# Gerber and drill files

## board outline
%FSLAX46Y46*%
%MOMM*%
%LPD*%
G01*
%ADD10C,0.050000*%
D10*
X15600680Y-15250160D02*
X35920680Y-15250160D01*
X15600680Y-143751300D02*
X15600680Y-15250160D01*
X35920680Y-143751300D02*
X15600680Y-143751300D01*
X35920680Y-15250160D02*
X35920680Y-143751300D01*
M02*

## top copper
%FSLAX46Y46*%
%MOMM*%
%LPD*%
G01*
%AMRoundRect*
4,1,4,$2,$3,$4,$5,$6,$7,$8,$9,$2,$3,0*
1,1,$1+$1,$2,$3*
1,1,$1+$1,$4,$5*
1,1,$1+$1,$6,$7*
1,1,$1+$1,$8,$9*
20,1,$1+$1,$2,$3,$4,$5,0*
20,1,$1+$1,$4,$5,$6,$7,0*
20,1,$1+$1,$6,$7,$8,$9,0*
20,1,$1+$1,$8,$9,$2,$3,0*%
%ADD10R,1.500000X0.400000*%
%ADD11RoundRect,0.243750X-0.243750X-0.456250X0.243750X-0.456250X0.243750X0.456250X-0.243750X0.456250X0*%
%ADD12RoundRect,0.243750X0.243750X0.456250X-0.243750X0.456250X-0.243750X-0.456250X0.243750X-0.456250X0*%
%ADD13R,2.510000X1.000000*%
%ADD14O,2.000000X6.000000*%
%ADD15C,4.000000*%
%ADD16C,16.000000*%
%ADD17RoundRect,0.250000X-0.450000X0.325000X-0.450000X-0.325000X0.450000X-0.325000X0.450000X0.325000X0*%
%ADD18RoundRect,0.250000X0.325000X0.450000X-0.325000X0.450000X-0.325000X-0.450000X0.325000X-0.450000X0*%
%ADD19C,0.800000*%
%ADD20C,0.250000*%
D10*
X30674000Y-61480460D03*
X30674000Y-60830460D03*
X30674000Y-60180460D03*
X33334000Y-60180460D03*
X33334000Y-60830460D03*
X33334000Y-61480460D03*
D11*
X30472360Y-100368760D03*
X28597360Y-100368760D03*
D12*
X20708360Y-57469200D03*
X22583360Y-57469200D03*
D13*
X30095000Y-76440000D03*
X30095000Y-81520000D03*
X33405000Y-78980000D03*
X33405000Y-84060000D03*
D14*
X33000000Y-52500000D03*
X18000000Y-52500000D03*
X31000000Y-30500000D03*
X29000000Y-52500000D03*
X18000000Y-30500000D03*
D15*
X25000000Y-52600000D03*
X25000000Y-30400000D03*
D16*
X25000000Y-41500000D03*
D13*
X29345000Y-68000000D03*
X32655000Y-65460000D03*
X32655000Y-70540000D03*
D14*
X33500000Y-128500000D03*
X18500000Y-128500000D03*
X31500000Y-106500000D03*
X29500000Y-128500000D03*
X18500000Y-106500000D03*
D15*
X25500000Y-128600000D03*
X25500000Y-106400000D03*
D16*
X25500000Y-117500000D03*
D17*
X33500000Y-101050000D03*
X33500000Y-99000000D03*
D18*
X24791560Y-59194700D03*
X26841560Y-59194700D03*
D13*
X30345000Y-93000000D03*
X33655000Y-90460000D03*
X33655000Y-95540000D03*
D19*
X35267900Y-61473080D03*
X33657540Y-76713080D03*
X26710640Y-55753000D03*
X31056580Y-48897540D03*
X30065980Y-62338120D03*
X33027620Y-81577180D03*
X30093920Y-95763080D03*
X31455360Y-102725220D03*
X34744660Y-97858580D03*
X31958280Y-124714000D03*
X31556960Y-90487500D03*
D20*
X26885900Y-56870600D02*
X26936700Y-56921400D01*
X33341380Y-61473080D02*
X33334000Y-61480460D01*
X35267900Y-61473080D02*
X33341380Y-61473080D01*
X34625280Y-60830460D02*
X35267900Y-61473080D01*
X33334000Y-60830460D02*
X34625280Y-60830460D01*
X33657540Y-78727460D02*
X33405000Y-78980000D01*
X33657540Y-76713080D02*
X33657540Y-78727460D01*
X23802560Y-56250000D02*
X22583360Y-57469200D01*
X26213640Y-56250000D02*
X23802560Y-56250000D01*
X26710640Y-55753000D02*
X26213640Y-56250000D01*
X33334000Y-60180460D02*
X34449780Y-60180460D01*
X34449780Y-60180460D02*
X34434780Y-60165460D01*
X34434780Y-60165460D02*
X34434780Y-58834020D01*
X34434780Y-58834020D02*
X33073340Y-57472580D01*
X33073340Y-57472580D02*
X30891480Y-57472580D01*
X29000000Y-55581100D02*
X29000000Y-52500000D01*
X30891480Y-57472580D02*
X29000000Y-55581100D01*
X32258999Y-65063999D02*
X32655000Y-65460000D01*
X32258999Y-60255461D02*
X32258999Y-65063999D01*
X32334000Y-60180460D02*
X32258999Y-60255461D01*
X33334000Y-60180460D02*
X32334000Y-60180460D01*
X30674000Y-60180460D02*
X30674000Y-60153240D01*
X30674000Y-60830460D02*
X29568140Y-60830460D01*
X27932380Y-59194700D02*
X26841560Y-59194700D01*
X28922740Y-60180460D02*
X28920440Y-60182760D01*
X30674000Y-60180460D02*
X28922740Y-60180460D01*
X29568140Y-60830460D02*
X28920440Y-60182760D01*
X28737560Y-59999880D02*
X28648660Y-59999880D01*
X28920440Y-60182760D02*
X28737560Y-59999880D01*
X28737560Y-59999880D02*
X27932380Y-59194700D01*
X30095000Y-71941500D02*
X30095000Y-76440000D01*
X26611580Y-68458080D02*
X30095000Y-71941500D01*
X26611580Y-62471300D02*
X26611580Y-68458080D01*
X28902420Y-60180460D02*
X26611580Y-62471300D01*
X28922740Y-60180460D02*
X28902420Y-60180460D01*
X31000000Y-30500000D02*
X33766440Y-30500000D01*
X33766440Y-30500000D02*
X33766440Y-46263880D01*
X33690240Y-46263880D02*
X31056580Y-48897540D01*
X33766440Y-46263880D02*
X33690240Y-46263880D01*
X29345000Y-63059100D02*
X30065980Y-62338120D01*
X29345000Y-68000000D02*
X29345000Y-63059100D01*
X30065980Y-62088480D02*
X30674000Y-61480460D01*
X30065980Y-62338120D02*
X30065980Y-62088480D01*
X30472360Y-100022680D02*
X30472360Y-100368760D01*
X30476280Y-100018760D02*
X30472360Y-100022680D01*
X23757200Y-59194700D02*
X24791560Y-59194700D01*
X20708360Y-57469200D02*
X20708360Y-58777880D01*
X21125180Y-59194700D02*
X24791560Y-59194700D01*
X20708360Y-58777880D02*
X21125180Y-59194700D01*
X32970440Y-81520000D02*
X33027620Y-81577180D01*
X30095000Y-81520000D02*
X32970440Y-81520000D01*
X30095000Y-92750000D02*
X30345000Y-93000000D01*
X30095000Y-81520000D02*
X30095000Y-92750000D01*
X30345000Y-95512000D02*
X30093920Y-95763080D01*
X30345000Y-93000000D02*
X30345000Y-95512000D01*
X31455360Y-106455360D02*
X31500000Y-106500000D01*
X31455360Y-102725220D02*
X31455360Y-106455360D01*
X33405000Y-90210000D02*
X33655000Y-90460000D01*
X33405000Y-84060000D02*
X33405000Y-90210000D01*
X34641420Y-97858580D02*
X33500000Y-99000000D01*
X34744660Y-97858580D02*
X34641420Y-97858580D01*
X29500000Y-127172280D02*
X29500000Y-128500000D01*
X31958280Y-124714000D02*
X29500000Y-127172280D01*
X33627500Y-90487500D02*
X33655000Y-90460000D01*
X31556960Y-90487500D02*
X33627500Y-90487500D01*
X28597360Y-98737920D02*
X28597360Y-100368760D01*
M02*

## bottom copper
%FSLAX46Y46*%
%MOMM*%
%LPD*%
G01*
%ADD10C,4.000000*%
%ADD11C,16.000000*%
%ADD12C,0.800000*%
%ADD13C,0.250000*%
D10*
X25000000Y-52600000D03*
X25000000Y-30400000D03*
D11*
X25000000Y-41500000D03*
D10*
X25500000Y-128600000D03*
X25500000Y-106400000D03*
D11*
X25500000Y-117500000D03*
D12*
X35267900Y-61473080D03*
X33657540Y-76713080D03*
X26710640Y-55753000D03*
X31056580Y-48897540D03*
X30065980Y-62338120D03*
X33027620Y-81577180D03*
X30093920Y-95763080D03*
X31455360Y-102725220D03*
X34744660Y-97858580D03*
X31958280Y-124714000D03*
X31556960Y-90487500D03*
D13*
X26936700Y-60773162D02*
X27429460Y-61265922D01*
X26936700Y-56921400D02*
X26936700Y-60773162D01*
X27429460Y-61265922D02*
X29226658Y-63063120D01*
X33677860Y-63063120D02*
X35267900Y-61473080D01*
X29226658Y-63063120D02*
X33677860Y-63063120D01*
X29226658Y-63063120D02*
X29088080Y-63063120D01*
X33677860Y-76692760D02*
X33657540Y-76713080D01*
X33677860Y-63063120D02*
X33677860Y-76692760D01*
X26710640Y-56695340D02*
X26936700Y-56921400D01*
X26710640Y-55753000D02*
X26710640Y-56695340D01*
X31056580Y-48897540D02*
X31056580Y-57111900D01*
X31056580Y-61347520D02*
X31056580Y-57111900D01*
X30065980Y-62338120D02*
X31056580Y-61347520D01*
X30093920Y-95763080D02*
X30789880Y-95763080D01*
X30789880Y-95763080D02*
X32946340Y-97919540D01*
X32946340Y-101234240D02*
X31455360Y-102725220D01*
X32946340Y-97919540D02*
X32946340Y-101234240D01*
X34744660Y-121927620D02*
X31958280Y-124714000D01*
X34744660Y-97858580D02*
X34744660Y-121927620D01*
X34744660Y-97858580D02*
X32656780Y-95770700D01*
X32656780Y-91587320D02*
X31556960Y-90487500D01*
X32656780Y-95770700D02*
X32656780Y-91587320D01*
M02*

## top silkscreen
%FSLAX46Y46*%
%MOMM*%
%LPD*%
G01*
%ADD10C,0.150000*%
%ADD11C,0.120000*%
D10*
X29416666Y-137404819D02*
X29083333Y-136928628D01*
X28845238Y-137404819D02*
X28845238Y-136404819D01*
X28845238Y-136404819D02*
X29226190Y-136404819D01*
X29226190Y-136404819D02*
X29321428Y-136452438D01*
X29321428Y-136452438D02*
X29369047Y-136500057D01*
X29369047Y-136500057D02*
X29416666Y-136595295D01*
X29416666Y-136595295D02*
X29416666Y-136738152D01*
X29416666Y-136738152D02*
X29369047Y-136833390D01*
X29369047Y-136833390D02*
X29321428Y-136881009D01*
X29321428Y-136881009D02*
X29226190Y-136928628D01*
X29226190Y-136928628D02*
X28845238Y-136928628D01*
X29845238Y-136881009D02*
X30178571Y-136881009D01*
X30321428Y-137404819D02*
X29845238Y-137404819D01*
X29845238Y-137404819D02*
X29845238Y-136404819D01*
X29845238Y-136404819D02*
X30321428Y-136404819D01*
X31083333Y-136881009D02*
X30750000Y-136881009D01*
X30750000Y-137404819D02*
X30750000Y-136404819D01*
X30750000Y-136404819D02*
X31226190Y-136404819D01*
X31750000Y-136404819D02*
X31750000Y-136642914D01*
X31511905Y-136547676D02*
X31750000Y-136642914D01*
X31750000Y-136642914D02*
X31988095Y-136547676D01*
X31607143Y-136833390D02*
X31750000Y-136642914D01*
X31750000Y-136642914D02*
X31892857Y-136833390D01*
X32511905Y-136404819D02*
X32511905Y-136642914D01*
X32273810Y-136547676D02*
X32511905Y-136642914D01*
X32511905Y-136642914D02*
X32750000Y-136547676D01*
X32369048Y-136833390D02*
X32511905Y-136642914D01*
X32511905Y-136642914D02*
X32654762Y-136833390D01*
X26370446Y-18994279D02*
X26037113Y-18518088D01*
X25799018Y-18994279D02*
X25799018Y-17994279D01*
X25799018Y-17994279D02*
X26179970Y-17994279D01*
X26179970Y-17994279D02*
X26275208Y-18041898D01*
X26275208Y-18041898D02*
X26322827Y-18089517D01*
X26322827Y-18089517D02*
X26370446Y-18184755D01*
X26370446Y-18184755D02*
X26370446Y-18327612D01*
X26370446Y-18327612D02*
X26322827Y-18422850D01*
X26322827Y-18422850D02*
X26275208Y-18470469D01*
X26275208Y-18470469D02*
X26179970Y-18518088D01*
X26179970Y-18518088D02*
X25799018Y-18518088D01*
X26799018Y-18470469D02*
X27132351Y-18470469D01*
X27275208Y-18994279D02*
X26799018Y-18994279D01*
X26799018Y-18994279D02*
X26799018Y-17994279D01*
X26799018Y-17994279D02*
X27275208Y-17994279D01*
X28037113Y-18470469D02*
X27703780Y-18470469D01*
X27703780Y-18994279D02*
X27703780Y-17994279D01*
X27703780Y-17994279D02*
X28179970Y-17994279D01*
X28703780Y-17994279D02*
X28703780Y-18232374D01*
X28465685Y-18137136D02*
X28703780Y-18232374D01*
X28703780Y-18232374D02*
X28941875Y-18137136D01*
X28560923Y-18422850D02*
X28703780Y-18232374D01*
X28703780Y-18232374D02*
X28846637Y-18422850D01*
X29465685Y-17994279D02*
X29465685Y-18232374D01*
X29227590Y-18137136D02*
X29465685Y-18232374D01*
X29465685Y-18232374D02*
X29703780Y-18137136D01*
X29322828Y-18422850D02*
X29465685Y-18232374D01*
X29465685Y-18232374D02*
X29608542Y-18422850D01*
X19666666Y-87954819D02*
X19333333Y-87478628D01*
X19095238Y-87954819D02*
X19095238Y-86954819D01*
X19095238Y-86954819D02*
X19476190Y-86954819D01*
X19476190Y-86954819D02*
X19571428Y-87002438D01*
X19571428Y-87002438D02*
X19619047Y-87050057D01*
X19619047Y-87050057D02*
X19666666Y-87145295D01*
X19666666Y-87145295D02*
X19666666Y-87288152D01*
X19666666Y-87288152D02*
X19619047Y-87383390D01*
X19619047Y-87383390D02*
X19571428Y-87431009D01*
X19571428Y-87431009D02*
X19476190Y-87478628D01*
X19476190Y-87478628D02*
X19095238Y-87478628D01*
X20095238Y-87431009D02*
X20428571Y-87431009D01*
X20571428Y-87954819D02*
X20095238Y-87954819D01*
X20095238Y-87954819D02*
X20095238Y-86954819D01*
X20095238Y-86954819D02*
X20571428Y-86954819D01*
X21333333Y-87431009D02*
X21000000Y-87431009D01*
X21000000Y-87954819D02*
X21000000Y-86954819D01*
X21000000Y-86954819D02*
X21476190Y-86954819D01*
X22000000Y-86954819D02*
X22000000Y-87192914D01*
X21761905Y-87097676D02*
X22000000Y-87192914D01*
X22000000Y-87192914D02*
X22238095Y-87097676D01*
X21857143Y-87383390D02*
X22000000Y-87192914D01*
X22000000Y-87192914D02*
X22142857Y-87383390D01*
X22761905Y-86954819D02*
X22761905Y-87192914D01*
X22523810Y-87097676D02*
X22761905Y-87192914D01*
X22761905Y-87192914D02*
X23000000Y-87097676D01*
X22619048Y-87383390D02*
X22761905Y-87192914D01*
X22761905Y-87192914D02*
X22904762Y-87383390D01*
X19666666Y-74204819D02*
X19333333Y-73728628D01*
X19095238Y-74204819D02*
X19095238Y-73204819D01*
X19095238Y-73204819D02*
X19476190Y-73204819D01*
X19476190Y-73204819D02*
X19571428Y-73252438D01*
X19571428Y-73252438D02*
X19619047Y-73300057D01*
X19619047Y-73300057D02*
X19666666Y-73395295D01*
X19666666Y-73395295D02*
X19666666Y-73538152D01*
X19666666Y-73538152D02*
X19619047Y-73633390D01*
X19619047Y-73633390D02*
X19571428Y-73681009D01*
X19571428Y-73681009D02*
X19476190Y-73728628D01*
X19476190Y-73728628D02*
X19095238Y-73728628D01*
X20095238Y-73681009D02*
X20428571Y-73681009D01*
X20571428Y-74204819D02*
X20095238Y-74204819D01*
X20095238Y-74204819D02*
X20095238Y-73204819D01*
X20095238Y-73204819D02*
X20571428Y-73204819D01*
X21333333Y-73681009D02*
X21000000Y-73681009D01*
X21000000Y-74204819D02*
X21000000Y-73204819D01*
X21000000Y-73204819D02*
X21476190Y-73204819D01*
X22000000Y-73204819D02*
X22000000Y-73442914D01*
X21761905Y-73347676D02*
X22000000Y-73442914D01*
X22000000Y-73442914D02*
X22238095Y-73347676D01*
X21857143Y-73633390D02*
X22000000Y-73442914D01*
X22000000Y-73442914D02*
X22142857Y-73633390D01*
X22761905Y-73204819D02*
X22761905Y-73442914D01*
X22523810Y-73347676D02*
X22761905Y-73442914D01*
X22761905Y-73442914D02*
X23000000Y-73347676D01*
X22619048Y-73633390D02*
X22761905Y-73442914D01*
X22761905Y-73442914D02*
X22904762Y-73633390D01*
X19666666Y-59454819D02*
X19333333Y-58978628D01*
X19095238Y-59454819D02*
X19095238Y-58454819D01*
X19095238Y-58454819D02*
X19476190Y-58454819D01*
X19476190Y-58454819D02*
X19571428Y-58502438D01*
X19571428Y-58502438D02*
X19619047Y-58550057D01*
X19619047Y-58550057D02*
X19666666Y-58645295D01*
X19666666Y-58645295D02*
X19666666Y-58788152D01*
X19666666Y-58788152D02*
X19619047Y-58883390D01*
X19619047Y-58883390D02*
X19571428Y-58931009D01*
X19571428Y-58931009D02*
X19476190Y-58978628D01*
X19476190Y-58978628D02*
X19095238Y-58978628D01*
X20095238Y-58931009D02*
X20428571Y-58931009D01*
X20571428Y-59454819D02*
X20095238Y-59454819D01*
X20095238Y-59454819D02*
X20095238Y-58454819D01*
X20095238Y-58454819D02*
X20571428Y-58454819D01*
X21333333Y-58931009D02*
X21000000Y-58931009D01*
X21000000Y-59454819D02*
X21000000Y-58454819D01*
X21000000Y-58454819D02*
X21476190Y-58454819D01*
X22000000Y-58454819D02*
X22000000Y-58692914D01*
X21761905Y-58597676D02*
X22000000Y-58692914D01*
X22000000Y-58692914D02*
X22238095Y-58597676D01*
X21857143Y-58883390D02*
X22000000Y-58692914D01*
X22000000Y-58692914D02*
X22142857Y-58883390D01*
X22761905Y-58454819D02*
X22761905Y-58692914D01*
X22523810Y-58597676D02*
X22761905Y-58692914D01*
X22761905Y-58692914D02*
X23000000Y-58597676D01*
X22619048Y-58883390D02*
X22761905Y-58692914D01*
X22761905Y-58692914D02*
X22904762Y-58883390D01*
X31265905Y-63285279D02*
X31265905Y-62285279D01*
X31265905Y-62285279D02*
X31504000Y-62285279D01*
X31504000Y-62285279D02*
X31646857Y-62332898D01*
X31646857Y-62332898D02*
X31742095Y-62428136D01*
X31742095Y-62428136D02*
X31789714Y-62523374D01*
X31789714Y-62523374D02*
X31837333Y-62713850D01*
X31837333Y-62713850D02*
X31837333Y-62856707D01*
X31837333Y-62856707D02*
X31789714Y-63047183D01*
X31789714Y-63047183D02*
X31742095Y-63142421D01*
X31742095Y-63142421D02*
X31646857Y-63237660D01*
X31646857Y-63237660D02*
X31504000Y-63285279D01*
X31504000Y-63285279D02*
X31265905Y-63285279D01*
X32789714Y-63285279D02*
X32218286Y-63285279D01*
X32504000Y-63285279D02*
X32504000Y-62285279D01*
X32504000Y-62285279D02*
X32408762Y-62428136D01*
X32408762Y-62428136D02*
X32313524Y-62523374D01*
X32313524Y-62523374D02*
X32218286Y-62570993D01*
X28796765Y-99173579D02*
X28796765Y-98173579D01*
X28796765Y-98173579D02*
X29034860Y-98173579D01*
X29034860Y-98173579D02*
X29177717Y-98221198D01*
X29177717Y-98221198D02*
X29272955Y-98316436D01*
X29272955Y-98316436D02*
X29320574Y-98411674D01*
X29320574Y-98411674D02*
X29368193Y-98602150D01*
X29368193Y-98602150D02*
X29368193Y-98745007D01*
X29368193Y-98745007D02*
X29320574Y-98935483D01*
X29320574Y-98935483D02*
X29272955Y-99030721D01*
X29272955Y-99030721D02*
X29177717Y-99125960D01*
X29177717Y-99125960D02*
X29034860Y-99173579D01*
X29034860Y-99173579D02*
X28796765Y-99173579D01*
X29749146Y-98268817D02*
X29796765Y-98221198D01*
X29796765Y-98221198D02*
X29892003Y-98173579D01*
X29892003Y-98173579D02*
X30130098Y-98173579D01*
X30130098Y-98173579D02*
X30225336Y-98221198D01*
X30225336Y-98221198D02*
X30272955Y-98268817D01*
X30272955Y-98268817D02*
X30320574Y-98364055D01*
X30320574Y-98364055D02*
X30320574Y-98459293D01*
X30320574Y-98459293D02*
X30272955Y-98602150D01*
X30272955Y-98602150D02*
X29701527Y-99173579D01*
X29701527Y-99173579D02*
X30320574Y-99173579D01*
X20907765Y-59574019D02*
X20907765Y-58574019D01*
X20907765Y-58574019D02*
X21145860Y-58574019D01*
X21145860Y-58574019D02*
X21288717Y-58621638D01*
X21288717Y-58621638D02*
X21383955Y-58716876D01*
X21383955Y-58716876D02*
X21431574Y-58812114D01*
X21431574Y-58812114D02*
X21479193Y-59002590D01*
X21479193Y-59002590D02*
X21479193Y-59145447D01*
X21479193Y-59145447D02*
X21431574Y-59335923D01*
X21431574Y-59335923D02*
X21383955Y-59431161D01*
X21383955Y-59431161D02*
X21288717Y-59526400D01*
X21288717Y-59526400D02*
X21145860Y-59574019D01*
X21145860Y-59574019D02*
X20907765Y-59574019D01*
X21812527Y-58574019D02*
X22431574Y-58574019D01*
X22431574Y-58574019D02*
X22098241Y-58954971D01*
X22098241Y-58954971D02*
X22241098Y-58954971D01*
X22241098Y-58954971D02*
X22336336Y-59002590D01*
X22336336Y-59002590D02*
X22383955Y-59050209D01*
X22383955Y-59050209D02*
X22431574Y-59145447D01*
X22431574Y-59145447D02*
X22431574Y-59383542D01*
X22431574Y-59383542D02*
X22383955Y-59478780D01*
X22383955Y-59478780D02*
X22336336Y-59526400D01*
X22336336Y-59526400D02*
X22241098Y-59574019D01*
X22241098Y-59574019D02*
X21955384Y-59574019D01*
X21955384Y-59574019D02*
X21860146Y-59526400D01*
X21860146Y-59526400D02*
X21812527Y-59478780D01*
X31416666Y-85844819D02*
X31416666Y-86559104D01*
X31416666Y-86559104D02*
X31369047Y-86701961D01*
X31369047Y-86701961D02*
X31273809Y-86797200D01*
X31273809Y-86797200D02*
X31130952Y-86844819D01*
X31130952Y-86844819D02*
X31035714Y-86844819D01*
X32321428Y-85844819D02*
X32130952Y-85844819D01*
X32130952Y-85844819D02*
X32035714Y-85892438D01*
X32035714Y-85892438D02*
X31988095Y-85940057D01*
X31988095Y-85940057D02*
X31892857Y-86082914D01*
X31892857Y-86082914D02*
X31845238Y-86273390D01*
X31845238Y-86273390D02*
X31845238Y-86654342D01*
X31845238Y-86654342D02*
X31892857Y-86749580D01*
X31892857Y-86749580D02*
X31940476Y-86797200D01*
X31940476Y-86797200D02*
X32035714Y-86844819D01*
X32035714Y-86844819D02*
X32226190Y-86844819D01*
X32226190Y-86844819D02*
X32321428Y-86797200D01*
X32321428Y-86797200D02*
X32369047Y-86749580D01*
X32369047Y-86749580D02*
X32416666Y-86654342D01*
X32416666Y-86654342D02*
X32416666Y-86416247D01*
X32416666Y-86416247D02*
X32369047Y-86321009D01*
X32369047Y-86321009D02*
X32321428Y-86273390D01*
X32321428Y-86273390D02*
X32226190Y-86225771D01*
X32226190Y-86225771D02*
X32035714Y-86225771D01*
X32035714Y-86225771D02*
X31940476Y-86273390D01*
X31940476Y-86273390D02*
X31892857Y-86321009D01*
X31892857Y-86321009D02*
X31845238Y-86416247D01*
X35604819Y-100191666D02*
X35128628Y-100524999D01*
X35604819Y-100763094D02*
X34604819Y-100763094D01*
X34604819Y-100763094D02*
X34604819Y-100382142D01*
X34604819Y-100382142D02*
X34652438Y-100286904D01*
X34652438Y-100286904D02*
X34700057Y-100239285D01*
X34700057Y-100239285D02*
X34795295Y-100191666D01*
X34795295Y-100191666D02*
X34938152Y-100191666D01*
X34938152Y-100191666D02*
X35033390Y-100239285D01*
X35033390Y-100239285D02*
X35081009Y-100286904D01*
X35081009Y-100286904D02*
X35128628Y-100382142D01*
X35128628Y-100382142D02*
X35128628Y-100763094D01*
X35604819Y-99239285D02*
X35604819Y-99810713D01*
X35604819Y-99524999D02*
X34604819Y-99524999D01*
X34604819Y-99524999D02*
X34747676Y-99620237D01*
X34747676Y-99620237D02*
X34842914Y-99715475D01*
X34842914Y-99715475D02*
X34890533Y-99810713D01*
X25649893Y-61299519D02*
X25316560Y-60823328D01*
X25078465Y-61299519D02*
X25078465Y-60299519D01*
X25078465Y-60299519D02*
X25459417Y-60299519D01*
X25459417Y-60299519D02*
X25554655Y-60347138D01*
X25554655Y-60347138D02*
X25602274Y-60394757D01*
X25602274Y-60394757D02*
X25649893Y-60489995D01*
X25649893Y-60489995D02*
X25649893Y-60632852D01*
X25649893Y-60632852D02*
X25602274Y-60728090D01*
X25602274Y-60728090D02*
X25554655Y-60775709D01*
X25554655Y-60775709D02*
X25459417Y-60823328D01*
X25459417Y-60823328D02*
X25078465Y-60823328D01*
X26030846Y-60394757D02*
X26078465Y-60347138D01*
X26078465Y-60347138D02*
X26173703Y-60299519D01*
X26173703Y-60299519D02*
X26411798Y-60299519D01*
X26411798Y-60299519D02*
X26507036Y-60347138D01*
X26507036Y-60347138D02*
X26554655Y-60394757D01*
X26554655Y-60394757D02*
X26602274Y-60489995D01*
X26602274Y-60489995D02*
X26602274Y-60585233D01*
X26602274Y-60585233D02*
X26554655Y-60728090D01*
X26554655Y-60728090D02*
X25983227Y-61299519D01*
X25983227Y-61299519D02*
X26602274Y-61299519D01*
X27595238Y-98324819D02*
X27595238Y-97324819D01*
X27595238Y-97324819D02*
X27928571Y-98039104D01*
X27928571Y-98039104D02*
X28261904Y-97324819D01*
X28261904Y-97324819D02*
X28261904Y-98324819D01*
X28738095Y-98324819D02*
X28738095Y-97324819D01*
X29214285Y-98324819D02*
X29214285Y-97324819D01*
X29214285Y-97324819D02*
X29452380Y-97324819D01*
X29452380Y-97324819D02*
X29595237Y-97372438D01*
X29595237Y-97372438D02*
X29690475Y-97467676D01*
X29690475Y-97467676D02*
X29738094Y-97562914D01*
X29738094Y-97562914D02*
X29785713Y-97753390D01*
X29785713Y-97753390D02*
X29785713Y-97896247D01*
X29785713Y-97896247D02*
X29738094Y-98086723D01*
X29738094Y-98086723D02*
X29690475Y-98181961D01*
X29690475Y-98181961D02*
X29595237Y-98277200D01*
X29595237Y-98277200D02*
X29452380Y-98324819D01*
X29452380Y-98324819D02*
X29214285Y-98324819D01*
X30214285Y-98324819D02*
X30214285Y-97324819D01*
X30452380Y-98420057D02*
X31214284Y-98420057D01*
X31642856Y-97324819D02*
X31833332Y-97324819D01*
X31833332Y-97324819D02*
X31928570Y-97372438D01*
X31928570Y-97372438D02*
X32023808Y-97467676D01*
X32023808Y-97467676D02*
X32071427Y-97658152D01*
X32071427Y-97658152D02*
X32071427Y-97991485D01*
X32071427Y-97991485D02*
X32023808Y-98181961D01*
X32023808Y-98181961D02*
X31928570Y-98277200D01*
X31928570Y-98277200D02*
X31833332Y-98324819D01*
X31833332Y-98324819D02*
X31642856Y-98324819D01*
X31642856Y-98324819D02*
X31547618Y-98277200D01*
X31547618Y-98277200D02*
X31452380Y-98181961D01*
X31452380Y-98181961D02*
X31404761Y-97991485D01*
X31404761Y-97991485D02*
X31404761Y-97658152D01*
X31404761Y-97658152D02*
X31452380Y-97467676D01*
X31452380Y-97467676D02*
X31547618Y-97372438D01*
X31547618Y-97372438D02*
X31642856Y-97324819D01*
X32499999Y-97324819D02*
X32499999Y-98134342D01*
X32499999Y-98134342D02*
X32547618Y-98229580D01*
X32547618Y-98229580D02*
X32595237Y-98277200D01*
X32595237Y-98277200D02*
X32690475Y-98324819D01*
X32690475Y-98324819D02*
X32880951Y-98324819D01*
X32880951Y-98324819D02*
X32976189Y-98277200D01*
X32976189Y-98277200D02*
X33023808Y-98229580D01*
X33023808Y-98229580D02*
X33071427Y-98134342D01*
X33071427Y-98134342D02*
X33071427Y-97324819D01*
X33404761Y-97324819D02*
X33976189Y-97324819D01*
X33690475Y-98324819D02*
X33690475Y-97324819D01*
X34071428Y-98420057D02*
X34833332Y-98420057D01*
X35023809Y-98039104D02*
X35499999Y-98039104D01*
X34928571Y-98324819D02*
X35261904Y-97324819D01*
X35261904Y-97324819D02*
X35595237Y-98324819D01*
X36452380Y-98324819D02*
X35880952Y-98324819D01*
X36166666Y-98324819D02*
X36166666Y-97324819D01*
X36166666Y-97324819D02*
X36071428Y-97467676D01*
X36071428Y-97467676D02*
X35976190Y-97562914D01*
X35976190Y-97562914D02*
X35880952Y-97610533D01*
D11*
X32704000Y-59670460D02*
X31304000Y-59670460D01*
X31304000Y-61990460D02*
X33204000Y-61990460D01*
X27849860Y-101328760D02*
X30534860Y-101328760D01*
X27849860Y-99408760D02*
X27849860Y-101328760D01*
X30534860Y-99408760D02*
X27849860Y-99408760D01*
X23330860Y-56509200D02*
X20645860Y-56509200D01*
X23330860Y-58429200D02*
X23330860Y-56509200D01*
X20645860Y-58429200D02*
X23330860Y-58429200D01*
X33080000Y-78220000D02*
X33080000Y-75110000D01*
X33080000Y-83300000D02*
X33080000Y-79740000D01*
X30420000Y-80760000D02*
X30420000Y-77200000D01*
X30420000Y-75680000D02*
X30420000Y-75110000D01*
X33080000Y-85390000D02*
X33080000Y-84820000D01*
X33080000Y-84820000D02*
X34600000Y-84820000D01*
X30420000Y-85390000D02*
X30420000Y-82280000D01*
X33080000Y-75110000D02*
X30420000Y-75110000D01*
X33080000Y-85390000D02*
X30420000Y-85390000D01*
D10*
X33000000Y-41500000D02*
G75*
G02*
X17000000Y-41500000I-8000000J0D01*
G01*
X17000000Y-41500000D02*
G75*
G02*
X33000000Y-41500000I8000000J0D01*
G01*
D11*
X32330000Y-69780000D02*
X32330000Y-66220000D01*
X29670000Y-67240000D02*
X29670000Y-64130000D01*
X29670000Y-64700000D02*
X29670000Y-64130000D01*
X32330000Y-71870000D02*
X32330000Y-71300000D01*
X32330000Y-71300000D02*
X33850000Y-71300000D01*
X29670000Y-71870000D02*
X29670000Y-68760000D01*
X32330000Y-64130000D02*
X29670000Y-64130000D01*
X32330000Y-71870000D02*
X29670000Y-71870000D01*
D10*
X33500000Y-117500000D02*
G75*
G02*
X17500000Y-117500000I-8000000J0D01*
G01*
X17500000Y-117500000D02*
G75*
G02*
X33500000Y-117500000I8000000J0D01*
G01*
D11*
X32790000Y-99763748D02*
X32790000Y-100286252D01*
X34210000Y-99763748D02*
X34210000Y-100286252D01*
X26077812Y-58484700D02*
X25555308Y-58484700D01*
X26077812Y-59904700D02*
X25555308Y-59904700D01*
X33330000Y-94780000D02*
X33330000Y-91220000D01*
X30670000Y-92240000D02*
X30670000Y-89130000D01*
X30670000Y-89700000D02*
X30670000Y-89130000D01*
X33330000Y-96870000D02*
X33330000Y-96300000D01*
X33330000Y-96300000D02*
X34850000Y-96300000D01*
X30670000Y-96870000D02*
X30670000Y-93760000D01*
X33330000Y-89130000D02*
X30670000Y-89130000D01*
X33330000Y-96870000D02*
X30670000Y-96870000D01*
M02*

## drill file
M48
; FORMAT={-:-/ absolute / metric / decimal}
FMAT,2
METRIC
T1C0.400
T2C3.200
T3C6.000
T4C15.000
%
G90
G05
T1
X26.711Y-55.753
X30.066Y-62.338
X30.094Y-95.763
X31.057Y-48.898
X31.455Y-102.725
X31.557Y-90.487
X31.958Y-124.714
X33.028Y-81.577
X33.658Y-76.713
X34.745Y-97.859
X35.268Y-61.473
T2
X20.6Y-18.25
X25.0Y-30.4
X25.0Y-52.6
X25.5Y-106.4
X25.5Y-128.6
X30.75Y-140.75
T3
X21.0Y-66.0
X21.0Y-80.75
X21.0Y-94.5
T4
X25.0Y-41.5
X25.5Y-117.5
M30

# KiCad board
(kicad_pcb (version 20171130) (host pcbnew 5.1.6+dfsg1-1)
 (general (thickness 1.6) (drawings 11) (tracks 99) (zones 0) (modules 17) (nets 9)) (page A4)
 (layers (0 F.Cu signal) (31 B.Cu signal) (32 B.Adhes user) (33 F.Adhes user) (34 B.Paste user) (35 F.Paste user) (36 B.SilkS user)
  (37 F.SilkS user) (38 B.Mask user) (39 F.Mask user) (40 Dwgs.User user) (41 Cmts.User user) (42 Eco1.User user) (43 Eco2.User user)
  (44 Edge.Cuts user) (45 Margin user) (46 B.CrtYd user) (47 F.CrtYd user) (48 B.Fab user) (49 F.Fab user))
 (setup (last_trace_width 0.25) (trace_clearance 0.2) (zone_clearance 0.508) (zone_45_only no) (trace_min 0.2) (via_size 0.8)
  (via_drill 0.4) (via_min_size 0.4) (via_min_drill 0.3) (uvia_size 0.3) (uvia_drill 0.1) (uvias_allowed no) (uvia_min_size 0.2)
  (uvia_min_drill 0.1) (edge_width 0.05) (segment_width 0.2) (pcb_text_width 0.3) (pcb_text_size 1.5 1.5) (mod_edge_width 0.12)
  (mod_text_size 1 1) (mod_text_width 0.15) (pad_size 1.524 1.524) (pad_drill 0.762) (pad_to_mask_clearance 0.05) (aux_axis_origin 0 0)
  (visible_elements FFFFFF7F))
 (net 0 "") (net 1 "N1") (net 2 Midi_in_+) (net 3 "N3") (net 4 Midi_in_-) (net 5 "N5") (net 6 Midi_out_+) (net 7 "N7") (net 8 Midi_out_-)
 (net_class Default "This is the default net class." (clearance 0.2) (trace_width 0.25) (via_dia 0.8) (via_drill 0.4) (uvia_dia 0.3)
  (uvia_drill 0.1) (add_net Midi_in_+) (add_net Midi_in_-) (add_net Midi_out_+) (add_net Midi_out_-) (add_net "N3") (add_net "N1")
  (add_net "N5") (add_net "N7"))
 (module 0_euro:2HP (layer F.Cu) (at 15.6 15)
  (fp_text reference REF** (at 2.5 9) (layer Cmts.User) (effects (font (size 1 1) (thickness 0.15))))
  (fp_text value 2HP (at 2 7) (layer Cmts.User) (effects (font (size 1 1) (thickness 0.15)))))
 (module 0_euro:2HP (layer F.Cu) (at 25.76 15)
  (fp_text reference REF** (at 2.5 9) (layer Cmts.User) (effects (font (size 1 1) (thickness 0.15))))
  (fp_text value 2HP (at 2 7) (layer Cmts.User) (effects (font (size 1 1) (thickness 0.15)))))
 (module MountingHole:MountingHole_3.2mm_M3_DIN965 (layer F.Cu) (at 30.75 140.75)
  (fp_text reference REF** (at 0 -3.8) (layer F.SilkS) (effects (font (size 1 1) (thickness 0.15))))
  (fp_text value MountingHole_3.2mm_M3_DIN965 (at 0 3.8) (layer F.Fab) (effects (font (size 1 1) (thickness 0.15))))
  (pad 1 np_thru_hole circle (at 0 0) (size 3.2 3.2) (drill 3.2) (layers *.Cu *.Mask)))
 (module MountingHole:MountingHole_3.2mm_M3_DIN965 (layer F.Cu) (at 20.6 18.25)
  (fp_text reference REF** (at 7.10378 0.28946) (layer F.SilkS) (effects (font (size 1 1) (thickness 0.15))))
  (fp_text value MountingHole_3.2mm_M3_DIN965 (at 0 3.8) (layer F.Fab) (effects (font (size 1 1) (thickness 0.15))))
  (pad 1 np_thru_hole circle (at 0 0) (size 3.2 3.2) (drill 3.2) (layers *.Cu *.Mask)))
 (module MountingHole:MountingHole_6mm (layer F.Cu) (at 21 94.5)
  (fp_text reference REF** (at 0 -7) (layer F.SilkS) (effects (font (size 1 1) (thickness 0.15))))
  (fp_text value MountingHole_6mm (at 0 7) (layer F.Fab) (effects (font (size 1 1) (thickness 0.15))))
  (pad 1 np_thru_hole circle (at 0 0) (size 6 6) (drill 6) (layers *.Cu *.Mask)))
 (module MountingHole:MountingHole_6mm (layer F.Cu) (at 21 80.75)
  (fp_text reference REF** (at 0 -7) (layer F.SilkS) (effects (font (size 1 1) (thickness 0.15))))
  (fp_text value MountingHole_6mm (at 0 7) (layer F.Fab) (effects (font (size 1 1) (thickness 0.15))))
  (pad 1 np_thru_hole circle (at 0 0) (size 6 6) (drill 6) (layers *.Cu *.Mask)))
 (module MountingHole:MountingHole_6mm (layer F.Cu) (at 21 66)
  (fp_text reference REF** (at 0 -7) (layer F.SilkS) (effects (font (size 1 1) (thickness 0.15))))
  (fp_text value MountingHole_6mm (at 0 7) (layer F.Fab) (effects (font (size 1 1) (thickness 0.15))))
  (pad 1 np_thru_hole circle (at 0 0) (size 6 6) (drill 6) (layers *.Cu *.Mask)))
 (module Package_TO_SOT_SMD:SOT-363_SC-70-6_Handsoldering (layer F.Cu) (at 32.004 60.83046 180)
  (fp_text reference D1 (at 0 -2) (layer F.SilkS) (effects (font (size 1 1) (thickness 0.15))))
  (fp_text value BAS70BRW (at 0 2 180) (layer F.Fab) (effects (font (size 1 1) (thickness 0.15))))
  (fp_line (start -0.7 1.16) (end 0.7 1.16) (layer F.SilkS) (width 0.12))
  (fp_line (start 0.7 -1.16) (end -1.2 -1.16) (layer F.SilkS) (width 0.12))
  (pad 6 smd rect (at 1.33 -0.65 180) (size 1.5 0.4) (layers F.Cu F.Paste F.Mask) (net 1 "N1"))
  (pad 5 smd rect (at 1.33 0 180) (size 1.5 0.4) (layers F.Cu F.Paste F.Mask) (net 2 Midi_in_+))
  (pad 4 smd rect (at 1.33 0.65 180) (size 1.5 0.4) (layers F.Cu F.Paste F.Mask) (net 2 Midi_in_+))
  (pad 3 smd rect (at -1.33 0.65 180) (size 1.5 0.4) (layers F.Cu F.Paste F.Mask) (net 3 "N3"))
  (pad 2 smd rect (at -1.33 0 180) (size 1.5 0.4) (layers F.Cu F.Paste F.Mask) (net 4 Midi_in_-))
  (pad 1 smd rect (at -1.33 -0.65 180) (size 1.5 0.4) (layers F.Cu F.Paste F.Mask) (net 4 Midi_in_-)))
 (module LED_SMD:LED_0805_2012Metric (layer F.Cu) (at 29.53486 100.36876)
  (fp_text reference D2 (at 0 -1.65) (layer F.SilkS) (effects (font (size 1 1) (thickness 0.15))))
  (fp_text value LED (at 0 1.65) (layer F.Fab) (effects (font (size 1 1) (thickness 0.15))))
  (fp_line (start -1.685 0.96) (end 1 0.96) (layer F.SilkS) (width 0.12))
  (fp_line (start -1.685 -0.96) (end -1.685 0.96) (layer F.SilkS) (width 0.12))
  (fp_line (start 1 -0.96) (end -1.685 -0.96) (layer F.SilkS) (width 0.12))
  (pad 2 smd roundrect (at 0.9375 0) (size 0.975 1.4) (layers F.Cu F.Paste F.Mask) (roundrect_rratio 0.25) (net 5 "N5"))
  (pad 1 smd roundrect (at -0.9375 0) (size 0.975 1.4) (layers F.Cu F.Paste F.Mask) (roundrect_rratio 0.25) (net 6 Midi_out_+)))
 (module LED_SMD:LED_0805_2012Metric (layer F.Cu) (at 21.64586 57.4692 180)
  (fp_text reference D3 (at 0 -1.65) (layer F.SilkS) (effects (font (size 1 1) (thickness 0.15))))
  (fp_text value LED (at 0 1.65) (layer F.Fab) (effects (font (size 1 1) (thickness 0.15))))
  (fp_line (start -1.685 0.96) (end 1 0.96) (layer F.SilkS) (width 0.12))
  (fp_line (start -1.685 -0.96) (end -1.685 0.96) (layer F.SilkS) (width 0.12))
  (fp_line (start 1 -0.96) (end -1.685 -0.96) (layer F.SilkS) (width 0.12))
  (pad 2 smd roundrect (at 0.9375 0 180) (size 0.975 1.4) (layers F.Cu F.Paste F.Mask) (roundrect_rratio 0.25) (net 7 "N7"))
  (pad 1 smd roundrect (at -0.9375 0 180) (size 0.975 1.4) (layers F.Cu F.Paste F.Mask) (roundrect_rratio 0.25) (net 4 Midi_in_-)))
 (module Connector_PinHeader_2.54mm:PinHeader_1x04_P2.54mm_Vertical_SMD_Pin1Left (layer F.Cu) (at 31.75 80.25 180)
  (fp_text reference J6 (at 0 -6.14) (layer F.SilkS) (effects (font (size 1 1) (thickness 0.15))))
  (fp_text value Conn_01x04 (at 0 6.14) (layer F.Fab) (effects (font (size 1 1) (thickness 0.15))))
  (fp_line (start -1.33 2.03) (end -1.33 5.14) (layer F.SilkS) (width 0.12))
  (fp_line (start -1.33 -3.05) (end -1.33 0.51) (layer F.SilkS) (width 0.12))
  (fp_line (start 1.33 -0.51) (end 1.33 3.05) (layer F.SilkS) (width 0.12))
  (fp_line (start 1.33 4.57) (end 1.33 5.14) (layer F.SilkS) (width 0.12))
  (fp_line (start -1.33 -5.14) (end -1.33 -4.57) (layer F.SilkS) (width 0.12))
  (fp_line (start -1.33 -4.57) (end -2.85 -4.57) (layer F.SilkS) (width 0.12))
  (fp_line (start 1.33 -5.14) (end 1.33 -2.03) (layer F.SilkS) (width 0.12))
  (fp_line (start -1.33 5.14) (end 1.33 5.14) (layer F.SilkS) (width 0.12))
  (fp_line (start -1.33 -5.14) (end 1.33 -5.14) (layer F.SilkS) (width 0.12))
  (pad 4 smd rect (at 1.655 3.81 180) (size 2.51 1) (layers F.Cu F.Paste F.Mask) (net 2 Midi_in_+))
  (pad 2 smd rect (at 1.655 -1.27 180) (size 2.51 1) (layers F.Cu F.Paste F.Mask) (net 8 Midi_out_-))
  (pad 3 smd rect (at -1.655 1.27 180) (size 2.51 1) (layers F.Cu F.Paste F.Mask) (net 4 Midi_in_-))
  (pad 1 smd rect (at -1.655 -3.81 180) (size 2.51 1) (layers F.Cu F.Paste F.Mask) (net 6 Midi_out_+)))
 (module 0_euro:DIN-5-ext (layer F.Cu) (at 25 41.5)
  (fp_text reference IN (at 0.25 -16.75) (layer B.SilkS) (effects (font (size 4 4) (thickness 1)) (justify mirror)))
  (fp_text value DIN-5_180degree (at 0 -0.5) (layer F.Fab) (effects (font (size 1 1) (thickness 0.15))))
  (fp_circle (center 0 0) (end 0 -8) (layer F.SilkS) (width 0.15))
  (pad 2 smd oval (at 8 11) (size 2 6) (layers F.Cu F.Paste F.Mask))
  (pad 1 smd oval (at -7 11) (size 2 6) (layers F.Cu F.Paste F.Mask))
  (pad 5 smd oval (at 6 -11) (size 2 6) (layers F.Cu F.Paste F.Mask) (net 1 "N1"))
  (pad 4 smd oval (at 4 11) (size 2 6) (layers F.Cu F.Paste F.Mask) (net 3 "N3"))
  (pad 3 smd oval (at -7 -11) (size 2 6) (layers F.Cu F.Paste F.Mask))
  (pad "" np_thru_hole circle (at 0 11.1) (size 4 4) (drill 3.2) (layers *.Cu *.Mask))
  (pad "" np_thru_hole circle (at 0 -11.1) (size 4 4) (drill 3.2) (layers *.Cu *.Mask))
  (pad "" np_thru_hole circle (at 0 0) (size 16 16) (drill 15) (layers *.Cu *.Mask)))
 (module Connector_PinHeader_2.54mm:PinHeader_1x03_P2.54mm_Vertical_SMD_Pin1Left (layer F.Cu) (at 31 68 180)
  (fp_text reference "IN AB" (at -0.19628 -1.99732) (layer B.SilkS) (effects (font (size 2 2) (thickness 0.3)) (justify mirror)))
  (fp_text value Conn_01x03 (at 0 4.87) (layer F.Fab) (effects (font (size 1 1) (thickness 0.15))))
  (fp_line (start -1.33 -1.78) (end -1.33 1.78) (layer F.SilkS) (width 0.12))
  (fp_line (start 1.33 0.76) (end 1.33 3.87) (layer F.SilkS) (width 0.12))
  (fp_line (start 1.33 3.3) (end 1.33 3.87) (layer F.SilkS) (width 0.12))
  (fp_line (start -1.33 -3.87) (end -1.33 -3.3) (layer F.SilkS) (width 0.12))
  (fp_line (start -1.33 -3.3) (end -2.85 -3.3) (layer F.SilkS) (width 0.12))
  (fp_line (start 1.33 -3.87) (end 1.33 -0.76) (layer F.SilkS) (width 0.12))
  (fp_line (start -1.33 3.87) (end 1.33 3.87) (layer F.SilkS) (width 0.12))
  (fp_line (start -1.33 -3.87) (end 1.33 -3.87) (layer F.SilkS) (width 0.12))
  (pad 2 smd rect (at 1.655 0 180) (size 2.51 1) (layers F.Cu F.Paste F.Mask) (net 1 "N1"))
  (pad 3 smd rect (at -1.655 2.54 180) (size 2.51 1) (layers F.Cu F.Paste F.Mask) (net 3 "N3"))
  (pad 1 smd rect (at -1.655 -2.54 180) (size 2.51 1) (layers F.Cu F.Paste F.Mask)))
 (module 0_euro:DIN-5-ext (layer F.Cu) (at 25.5 117.5)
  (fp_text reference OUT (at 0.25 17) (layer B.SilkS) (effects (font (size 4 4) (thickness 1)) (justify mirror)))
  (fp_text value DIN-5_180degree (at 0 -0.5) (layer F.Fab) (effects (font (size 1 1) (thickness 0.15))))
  (fp_circle (center 0 0) (end 0 -8) (layer F.SilkS) (width 0.15))
  (pad 2 smd oval (at 8 11) (size 2 6) (layers F.Cu F.Paste F.Mask))
  (pad 1 smd oval (at -7 11) (size 2 6) (layers F.Cu F.Paste F.Mask))
  (pad 5 smd oval (at 6 -11) (size 2 6) (layers F.Cu F.Paste F.Mask) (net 8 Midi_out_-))
  (pad 4 smd oval (at 4 11) (size 2 6) (layers F.Cu F.Paste F.Mask) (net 6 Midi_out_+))
  (pad 3 smd oval (at -7 -11) (size 2 6) (layers F.Cu F.Paste F.Mask))
  (pad "" np_thru_hole circle (at 0 11.1) (size 4 4) (drill 3.2) (layers *.Cu *.Mask))
  (pad "" np_thru_hole circle (at 0 -11.1) (size 4 4) (drill 3.2) (layers *.Cu *.Mask))
  (pad "" np_thru_hole circle (at 0 0) (size 16 16) (drill 15) (layers *.Cu *.Mask)))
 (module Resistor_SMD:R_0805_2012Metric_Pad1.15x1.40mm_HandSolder (layer F.Cu) (at 33.5 100.025 270)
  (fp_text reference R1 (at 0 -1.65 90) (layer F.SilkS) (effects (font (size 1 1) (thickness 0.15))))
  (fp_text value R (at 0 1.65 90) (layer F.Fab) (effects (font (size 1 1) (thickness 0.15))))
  (fp_line (start -0.261252 0.71) (end 0.261252 0.71) (layer F.SilkS) (width 0.12))
  (fp_line (start -0.261252 -0.71) (end 0.261252 -0.71) (layer F.SilkS) (width 0.12))
  (pad 2 smd roundrect (at 1.025 0 270) (size 1.15 1.4) (layers F.Cu F.Paste F.Mask) (roundrect_rratio 0.217391) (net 5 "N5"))
  (pad 1 smd roundrect (at -1.025 0 270) (size 1.15 1.4) (layers F.Cu F.Paste F.Mask) (roundrect_rratio 0.217391) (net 6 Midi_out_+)))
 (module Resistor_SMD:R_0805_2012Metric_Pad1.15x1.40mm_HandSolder (layer F.Cu) (at 25.81656 59.1947 180)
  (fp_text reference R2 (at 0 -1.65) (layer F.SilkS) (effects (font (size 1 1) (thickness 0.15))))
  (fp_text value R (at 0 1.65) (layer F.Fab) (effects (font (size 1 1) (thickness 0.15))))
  (fp_line (start -0.261252 0.71) (end 0.261252 0.71) (layer F.SilkS) (width 0.12))
  (fp_line (start -0.261252 -0.71) (end 0.261252 -0.71) (layer F.SilkS) (width 0.12))
  (pad 2 smd roundrect (at 1.025 0 180) (size 1.15 1.4) (layers F.Cu F.Paste F.Mask) (roundrect_rratio 0.217391) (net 7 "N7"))
  (pad 1 smd roundrect (at -1.025 0 180) (size 1.15 1.4) (layers F.Cu F.Paste F.Mask) (roundrect_rratio 0.217391) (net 2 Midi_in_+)))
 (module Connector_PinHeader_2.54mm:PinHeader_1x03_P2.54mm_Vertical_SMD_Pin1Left (layer F.Cu) (at 32 93 180)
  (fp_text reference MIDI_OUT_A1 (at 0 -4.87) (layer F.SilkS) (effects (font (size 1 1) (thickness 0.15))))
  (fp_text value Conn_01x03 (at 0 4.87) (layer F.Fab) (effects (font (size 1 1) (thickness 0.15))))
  (fp_line (start -1.33 -1.78) (end -1.33 1.78) (layer F.SilkS) (width 0.12))
  (fp_line (start 1.33 0.76) (end 1.33 3.87) (layer F.SilkS) (width 0.12))
  (fp_line (start 1.33 3.3) (end 1.33 3.87) (layer F.SilkS) (width 0.12))
  (fp_line (start -1.33 -3.87) (end -1.33 -3.3) (layer F.SilkS) (width 0.12))
  (fp_line (start -1.33 -3.3) (end -2.85 -3.3) (layer F.SilkS) (width 0.12))
  (fp_line (start 1.33 -3.87) (end 1.33 -0.76) (layer F.SilkS) (width 0.12))
  (fp_line (start -1.33 3.87) (end 1.33 3.87) (layer F.SilkS) (width 0.12))
  (fp_line (start -1.33 -3.87) (end 1.33 -3.87) (layer F.SilkS) (width 0.12))
  (pad 2 smd rect (at 1.655 0 180) (size 2.51 1) (layers F.Cu F.Paste F.Mask) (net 8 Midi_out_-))
  (pad 3 smd rect (at -1.655 2.54 180) (size 2.51 1) (layers F.Cu F.Paste F.Mask) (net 6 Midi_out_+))
  (pad 1 smd rect (at -1.655 -2.54 180) (size 2.51 1) (layers F.Cu F.Paste F.Mask)))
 (gr_line (start 15.60068 15.25016) (end 35.92068 15.25016) (layer Edge.Cuts) (width 0.05))
 (gr_line (start 15.60068 143.7513) (end 15.60068 15.25016) (layer Edge.Cuts) (width 0.05))
 (gr_line (start 35.92068 143.7513) (end 15.60068 143.7513) (layer Edge.Cuts) (width 0.05))
 (gr_line (start 35.92068 15.25016) (end 35.92068 143.7513) (layer Edge.Cuts) (width 0.05))
 (segment (start 26.8859 56.8706) (end 26.9367 56.9214) (width 0.25) (layer F.Cu) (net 4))
 (segment (start 26.9367 60.773162) (end 27.42946 61.265922) (width 0.25) (layer B.Cu) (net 4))
 (segment (start 26.9367 56.9214) (end 26.9367 60.773162) (width 0.25) (layer B.Cu) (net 4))
 (segment (start 27.42946 61.265922) (end 29.226658 63.06312) (width 0.25) (layer B.Cu) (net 4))
 (via (at 35.2679 61.47308) (size 0.8) (drill 0.4) (layers F.Cu B.Cu) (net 4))
 (segment (start 33.67786 63.06312) (end 35.2679 61.47308) (width 0.25) (layer B.Cu) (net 4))
 (segment (start 29.226658 63.06312) (end 33.67786 63.06312) (width 0.25) (layer B.Cu) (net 4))
 (segment (start 33.34138 61.47308) (end 33.334 61.48046) (width 0.25) (layer F.Cu) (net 4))
 (segment (start 35.2679 61.47308) (end 33.34138 61.47308) (width 0.25) (layer F.Cu) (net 4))
 (segment (start 34.62528 60.83046) (end 35.2679 61.47308) (width 0.25) (layer F.Cu) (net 4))
 (segment (start 33.334 60.83046) (end 34.62528 60.83046) (width 0.25) (layer F.Cu) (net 4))
 (segment (start 29.226658 63.06312) (end 29.08808 63.06312) (width 0.25) (layer B.Cu) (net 4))
 (via (at 33.65754 76.71308) (size 0.8) (drill 0.4) (layers F.Cu B.Cu) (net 4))
 (segment (start 33.67786 76.69276) (end 33.65754 76.71308) (width 0.25) (layer B.Cu) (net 4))
 (segment (start 33.67786 63.06312) (end 33.67786 76.69276) (width 0.25) (layer B.Cu) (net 4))
 (segment (start 33.65754 78.72746) (end 33.405 78.98) (width 0.25) (layer F.Cu) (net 4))
 (segment (start 33.65754 76.71308) (end 33.65754 78.72746) (width 0.25) (layer F.Cu) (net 4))
 (via (at 26.71064 55.753) (size 0.8) (drill 0.4) (layers F.Cu B.Cu) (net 4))
 (segment (start 26.71064 56.69534) (end 26.9367 56.9214) (width 0.25) (layer B.Cu) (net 4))
 (segment (start 26.71064 55.753) (end 26.71064 56.69534) (width 0.25) (layer B.Cu) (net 4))
 (segment (start 23.80256 56.25) (end 22.58336 57.4692) (width 0.25) (layer F.Cu) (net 4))
 (segment (start 26.21364 56.25) (end 23.80256 56.25) (width 0.25) (layer F.Cu) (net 4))
 (segment (start 26.71064 55.753) (end 26.21364 56.25) (width 0.25) (layer F.Cu) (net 4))
 (segment (start 33.334 60.18046) (end 34.44978 60.18046) (width 0.25) (layer F.Cu) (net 3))
 (segment (start 34.44978 60.18046) (end 34.43478 60.16546) (width 0.25) (layer F.Cu) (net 3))
 (segment (start 34.43478 60.16546) (end 34.43478 58.83402) (width 0.25) (layer F.Cu) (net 3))
 (segment (start 34.43478 58.83402) (end 33.07334 57.47258) (width 0.25) (layer F.Cu) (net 3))
 (segment (start 33.07334 57.47258) (end 30.89148 57.47258) (width 0.25) (layer F.Cu) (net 3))
 (segment (start 29 55.5811) (end 29 52.5) (width 0.25) (layer F.Cu) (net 3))
 (segment (start 30.89148 57.47258) (end 29 55.5811) (width 0.25) (layer F.Cu) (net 3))
 (segment (start 32.258999 65.063999) (end 32.655 65.46) (width 0.25) (layer F.Cu) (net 3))
 (segment (start 32.258999 60.255461) (end 32.258999 65.063999) (width 0.25) (layer F.Cu) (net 3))
 (segment (start 32.334 60.18046) (end 32.258999 60.255461) (width 0.25) (layer F.Cu) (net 3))
 (segment (start 33.334 60.18046) (end 32.334 60.18046) (width 0.25) (layer F.Cu) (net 3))
 (segment (start 30.674 60.18046) (end 30.674 60.15324) (width 0.25) (layer F.Cu) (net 2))
 (segment (start 30.674 60.83046) (end 29.56814 60.83046) (width 0.25) (layer F.Cu) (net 2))
 (segment (start 27.93238 59.1947) (end 26.84156 59.1947) (width 0.25) (layer F.Cu) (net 2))
 (segment (start 28.92274 60.18046) (end 28.92044 60.18276) (width 0.25) (layer F.Cu) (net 2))
 (segment (start 30.674 60.18046) (end 28.92274 60.18046) (width 0.25) (layer F.Cu) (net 2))
 (segment (start 29.56814 60.83046) (end 28.92044 60.18276) (width 0.25) (layer F.Cu) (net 2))
 (segment (start 28.73756 59.99988) (end 28.64866 59.99988) (width 0.25) (layer F.Cu) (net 2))
 (segment (start 28.92044 60.18276) (end 28.73756 59.99988) (width 0.25) (layer F.Cu) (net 2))
 (segment (start 28.73756 59.99988) (end 27.93238 59.1947) (width 0.25) (layer F.Cu) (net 2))
 (segment (start 30.095 71.9415) (end 30.095 76.44) (width 0.25) (layer F.Cu) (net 2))
 (segment (start 26.61158 68.45808) (end 30.095 71.9415) (width 0.25) (layer F.Cu) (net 2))
 (segment (start 26.61158 62.4713) (end 26.61158 68.45808) (width 0.25) (layer F.Cu) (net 2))
 (segment (start 28.90242 60.18046) (end 26.61158 62.4713) (width 0.25) (layer F.Cu) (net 2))
 (segment (start 28.92274 60.18046) (end 28.90242 60.18046) (width 0.25) (layer F.Cu) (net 2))
 (segment (start 31 30.5) (end 33.76644 30.5) (width 0.25) (layer F.Cu) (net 1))
 (segment (start 33.76644 30.5) (end 33.76644 46.26388) (width 0.25) (layer F.Cu) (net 1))
 (via (at 31.05658 48.89754) (size 0.8) (drill 0.4) (layers F.Cu B.Cu) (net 1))
 (segment (start 33.69024 46.26388) (end 31.05658 48.89754) (width 0.25) (layer F.Cu) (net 1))
 (segment (start 33.76644 46.26388) (end 33.69024 46.26388) (width 0.25) (layer F.Cu) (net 1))
 (segment (start 31.05658 48.89754) (end 31.05658 57.1119) (width 0.25) (layer B.Cu) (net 1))
 (via (at 30.06598 62.33812) (size 0.8) (drill 0.4) (layers F.Cu B.Cu) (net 1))
 (segment (start 29.345 63.0591) (end 30.06598 62.33812) (width 0.25) (layer F.Cu) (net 1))
 (segment (start 29.345 68) (end 29.345 63.0591) (width 0.25) (layer F.Cu) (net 1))
 (segment (start 31.05658 61.34752) (end 31.05658 57.1119) (width 0.25) (layer B.Cu) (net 1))
 (segment (start 30.06598 62.33812) (end 31.05658 61.34752) (width 0.25) (layer B.Cu) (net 1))
 (segment (start 30.06598 62.08848) (end 30.674 61.48046) (width 0.25) (layer F.Cu) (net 1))
 (segment (start 30.06598 62.33812) (end 30.06598 62.08848) (width 0.25) (layer F.Cu) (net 1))
 (segment (start 30.47236 100.02268) (end 30.47236 100.36876) (width 0.25) (layer F.Cu) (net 5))
 (segment (start 30.47628 100.01876) (end 30.47236 100.02268) (width 0.25) (layer F.Cu) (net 5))
 (segment (start 23.7572 59.1947) (end 24.79156 59.1947) (width 0.25) (layer F.Cu) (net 7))
 (segment (start 20.70836 57.4692) (end 20.70836 58.77788) (width 0.25) (layer F.Cu) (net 7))
 (segment (start 21.12518 59.1947) (end 24.79156 59.1947) (width 0.25) (layer F.Cu) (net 7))
 (segment (start 20.70836 58.77788) (end 21.12518 59.1947) (width 0.25) (layer F.Cu) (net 7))
 (via (at 33.02762 81.57718) (size 0.8) (drill 0.4) (layers F.Cu B.Cu) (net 8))
 (segment (start 32.97044 81.52) (end 33.02762 81.57718) (width 0.25) (layer F.Cu) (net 8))
 (segment (start 30.095 81.52) (end 32.97044 81.52) (width 0.25) (layer F.Cu) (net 8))
 (segment (start 30.095 92.75) (end 30.345 93) (width 0.25) (layer F.Cu) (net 8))
 (segment (start 30.095 81.52) (end 30.095 92.75) (width 0.25) (layer F.Cu) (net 8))
 (via (at 30.09392 95.76308) (size 0.8) (drill 0.4) (layers F.Cu B.Cu) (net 8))
 (segment (start 30.345 95.512) (end 30.09392 95.76308) (width 0.25) (layer F.Cu) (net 8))
 (segment (start 30.345 93) (end 30.345 95.512) (width 0.25) (layer F.Cu) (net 8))
 (via (at 31.45536 102.72522) (size 0.8) (drill 0.4) (layers F.Cu B.Cu) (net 8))
 (segment (start 31.45536 106.45536) (end 31.5 106.5) (width 0.25) (layer F.Cu) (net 8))
 (segment (start 31.45536 102.72522) (end 31.45536 106.45536) (width 0.25) (layer F.Cu) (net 8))
 (segment (start 30.09392 95.76308) (end 30.78988 95.76308) (width 0.25) (layer B.Cu) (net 8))
 (segment (start 30.78988 95.76308) (end 32.94634 97.91954) (width 0.25) (layer B.Cu) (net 8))
 (segment (start 32.94634 101.23424) (end 31.45536 102.72522) (width 0.25) (layer B.Cu) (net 8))
 (segment (start 32.94634 97.91954) (end 32.94634 101.23424) (width 0.25) (layer B.Cu) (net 8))
 (segment (start 33.405 90.21) (end 33.655 90.46) (width 0.25) (layer F.Cu) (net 6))
 (segment (start 33.405 84.06) (end 33.405 90.21) (width 0.25) (layer F.Cu) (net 6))
 (via (at 34.74466 97.85858) (size 0.8) (drill 0.4) (layers F.Cu B.Cu) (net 6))
 (segment (start 34.64142 97.85858) (end 33.5 99) (width 0.25) (layer F.Cu) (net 6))
 (segment (start 34.74466 97.85858) (end 34.64142 97.85858) (width 0.25) (layer F.Cu) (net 6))
 (via (at 31.95828 124.714) (size 0.8) (drill 0.4) (layers F.Cu B.Cu) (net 6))
 (segment (start 34.74466 121.92762) (end 31.95828 124.714) (width 0.25) (layer B.Cu) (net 6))
 (segment (start 34.74466 97.85858) (end 34.74466 121.92762) (width 0.25) (layer B.Cu) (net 6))
 (segment (start 29.5 127.17228) (end 29.5 128.5) (width 0.25) (layer F.Cu) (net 6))
 (segment (start 31.95828 124.714) (end 29.5 127.17228) (width 0.25) (layer F.Cu) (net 6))
 (segment (start 34.74466 97.85858) (end 32.65678 95.7707) (width 0.25) (layer B.Cu) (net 6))
 (via (at 31.55696 90.4875) (size 0.8) (drill 0.4) (layers F.Cu B.Cu) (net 6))
 (segment (start 32.65678 91.58732) (end 31.55696 90.4875) (width 0.25) (layer B.Cu) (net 6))
 (segment (start 32.65678 95.7707) (end 32.65678 91.58732) (width 0.25) (layer B.Cu) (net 6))
 (segment (start 33.6275 90.4875) (end 33.655 90.46) (width 0.25) (layer F.Cu) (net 6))
 (segment (start 31.55696 90.4875) (end 33.6275 90.4875) (width 0.25) (layer F.Cu) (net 6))
 (segment (start 28.59736 98.73792) (end 28.59736 100.36876) (width 0.25) (layer F.Cu) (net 6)))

